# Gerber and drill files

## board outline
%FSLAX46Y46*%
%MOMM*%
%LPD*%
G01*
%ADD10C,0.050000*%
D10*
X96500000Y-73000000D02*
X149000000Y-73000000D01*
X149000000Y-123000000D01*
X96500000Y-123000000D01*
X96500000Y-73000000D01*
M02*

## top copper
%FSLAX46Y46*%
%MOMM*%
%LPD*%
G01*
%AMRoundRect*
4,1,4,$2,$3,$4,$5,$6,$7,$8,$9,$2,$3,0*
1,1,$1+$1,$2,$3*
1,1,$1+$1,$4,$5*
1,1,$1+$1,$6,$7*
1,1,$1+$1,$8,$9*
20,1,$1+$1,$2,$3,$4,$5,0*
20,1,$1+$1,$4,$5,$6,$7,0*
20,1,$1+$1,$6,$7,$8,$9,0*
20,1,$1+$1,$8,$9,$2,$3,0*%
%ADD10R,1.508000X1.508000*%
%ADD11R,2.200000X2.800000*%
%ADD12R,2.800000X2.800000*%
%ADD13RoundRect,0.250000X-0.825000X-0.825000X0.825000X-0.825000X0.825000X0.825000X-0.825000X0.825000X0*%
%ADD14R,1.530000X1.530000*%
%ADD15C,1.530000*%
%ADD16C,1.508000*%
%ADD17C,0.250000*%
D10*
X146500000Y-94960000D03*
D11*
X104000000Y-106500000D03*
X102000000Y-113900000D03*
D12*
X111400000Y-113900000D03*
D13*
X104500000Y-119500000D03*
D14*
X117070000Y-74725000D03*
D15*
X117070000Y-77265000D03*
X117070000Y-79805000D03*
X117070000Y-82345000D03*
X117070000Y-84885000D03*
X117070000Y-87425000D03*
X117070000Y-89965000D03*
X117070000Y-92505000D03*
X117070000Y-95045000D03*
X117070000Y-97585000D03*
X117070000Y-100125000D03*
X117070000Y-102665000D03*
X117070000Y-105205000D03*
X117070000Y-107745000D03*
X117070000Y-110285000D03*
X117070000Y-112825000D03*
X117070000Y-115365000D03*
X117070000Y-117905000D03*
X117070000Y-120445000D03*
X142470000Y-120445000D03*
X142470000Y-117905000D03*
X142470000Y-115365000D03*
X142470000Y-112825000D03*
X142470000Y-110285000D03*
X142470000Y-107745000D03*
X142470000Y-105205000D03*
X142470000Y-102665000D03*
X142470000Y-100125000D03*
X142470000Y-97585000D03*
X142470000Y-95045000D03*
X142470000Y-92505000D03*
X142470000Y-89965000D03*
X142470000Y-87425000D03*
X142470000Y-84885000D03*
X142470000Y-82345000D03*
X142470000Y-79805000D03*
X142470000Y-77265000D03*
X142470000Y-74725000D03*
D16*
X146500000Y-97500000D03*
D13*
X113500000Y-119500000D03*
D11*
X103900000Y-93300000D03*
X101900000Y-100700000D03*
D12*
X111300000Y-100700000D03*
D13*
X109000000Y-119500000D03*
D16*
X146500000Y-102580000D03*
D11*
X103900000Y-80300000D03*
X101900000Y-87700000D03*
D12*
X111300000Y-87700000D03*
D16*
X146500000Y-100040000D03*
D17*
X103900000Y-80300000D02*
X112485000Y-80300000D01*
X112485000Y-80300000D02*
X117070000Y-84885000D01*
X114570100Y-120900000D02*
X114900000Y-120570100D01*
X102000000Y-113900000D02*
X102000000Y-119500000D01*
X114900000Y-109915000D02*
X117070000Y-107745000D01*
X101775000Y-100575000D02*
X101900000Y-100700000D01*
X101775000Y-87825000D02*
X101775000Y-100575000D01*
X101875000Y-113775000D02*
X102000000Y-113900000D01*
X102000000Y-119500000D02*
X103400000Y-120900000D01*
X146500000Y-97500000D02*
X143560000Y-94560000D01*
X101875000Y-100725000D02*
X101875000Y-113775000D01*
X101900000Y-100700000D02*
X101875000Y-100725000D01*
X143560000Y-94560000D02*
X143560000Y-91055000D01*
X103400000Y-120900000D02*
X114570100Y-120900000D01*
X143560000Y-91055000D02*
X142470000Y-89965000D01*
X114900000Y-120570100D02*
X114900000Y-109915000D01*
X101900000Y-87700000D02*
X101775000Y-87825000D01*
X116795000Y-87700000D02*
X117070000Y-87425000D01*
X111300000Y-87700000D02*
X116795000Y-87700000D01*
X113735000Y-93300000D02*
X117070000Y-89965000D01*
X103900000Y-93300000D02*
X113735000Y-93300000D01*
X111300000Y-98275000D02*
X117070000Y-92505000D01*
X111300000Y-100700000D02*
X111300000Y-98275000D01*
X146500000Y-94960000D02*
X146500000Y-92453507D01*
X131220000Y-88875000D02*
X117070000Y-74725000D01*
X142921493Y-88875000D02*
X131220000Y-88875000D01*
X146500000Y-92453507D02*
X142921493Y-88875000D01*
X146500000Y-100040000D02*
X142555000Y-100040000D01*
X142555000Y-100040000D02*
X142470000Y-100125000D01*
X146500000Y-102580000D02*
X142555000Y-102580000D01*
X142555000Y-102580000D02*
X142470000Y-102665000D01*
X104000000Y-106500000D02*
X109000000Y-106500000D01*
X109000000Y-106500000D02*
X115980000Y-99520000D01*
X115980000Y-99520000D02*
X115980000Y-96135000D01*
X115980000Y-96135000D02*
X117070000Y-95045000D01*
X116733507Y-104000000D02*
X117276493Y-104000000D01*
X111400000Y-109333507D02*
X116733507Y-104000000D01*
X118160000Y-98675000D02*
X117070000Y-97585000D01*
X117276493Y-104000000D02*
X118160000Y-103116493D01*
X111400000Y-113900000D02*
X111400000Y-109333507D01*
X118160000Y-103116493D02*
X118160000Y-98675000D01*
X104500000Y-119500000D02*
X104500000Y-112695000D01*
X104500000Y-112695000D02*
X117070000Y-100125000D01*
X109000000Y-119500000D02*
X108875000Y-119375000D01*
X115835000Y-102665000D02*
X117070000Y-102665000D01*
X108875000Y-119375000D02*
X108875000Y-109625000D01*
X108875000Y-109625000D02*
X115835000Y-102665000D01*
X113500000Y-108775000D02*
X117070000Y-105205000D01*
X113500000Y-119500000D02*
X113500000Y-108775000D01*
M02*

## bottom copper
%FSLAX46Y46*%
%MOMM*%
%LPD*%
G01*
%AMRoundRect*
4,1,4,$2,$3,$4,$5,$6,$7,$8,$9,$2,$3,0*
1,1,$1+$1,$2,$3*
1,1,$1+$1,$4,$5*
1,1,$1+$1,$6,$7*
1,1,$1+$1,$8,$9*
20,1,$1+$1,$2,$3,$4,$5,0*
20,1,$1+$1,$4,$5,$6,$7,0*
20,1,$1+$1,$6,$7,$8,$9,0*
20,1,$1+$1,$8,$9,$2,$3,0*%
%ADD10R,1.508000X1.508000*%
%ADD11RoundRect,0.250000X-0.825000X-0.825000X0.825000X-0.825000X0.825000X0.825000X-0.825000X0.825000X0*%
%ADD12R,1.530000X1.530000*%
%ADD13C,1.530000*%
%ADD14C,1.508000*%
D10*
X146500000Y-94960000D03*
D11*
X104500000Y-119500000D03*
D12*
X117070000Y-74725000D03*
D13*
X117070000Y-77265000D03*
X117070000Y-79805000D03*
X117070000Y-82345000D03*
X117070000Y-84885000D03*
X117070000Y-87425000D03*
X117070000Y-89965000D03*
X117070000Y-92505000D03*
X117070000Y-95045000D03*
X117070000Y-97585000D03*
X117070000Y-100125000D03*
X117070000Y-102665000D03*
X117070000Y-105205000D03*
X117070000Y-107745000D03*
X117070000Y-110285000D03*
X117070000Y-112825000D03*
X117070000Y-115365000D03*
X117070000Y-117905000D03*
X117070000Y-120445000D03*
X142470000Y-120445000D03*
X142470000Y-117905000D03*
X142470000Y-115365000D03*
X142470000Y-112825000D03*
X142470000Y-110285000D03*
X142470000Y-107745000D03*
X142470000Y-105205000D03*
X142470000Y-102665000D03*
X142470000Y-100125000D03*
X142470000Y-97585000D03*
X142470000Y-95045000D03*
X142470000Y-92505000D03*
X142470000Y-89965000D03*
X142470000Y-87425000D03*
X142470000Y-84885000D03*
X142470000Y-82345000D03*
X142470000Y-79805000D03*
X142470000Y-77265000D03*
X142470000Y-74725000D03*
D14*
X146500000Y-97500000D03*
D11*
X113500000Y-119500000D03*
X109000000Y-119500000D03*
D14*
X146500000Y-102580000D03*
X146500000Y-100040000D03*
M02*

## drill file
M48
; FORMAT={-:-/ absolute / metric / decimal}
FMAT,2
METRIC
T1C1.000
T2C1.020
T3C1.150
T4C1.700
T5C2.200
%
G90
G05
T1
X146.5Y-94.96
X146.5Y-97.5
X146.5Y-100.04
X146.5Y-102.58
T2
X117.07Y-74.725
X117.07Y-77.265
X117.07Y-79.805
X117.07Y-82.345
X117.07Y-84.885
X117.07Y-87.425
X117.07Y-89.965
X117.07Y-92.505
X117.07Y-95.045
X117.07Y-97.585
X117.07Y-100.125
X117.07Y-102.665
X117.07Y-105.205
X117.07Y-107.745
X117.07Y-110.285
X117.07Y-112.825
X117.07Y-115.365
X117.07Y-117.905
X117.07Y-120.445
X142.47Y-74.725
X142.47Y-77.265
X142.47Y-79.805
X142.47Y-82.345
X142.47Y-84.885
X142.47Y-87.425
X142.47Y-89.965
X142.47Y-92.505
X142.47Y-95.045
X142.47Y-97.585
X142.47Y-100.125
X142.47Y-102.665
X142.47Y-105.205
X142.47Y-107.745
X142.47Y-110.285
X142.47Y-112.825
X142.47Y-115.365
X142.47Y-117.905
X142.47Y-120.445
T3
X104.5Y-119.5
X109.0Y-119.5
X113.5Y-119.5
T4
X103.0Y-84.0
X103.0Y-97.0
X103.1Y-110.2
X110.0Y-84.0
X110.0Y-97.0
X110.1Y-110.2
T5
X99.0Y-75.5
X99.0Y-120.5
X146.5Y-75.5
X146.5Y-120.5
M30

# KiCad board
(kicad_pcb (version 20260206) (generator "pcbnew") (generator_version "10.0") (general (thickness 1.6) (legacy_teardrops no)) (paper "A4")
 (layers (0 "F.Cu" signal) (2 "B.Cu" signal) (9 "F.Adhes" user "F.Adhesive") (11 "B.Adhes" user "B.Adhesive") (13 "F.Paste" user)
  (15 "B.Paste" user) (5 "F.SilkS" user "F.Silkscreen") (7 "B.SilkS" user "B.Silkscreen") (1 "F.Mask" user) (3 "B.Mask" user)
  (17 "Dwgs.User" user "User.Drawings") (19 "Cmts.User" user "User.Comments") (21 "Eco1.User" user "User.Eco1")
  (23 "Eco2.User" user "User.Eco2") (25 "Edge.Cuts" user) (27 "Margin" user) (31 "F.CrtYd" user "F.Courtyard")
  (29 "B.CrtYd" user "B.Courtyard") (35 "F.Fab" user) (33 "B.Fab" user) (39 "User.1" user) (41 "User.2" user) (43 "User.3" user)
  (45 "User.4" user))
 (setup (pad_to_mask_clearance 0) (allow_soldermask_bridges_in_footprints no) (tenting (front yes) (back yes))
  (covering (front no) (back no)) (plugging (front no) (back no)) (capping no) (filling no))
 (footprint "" (layer "F.Cu") (at 146.5 94.96 -90)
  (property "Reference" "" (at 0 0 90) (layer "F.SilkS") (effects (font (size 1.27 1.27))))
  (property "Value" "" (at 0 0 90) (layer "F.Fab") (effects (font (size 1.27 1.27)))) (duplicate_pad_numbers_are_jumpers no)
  (pad "1" thru_hole rect (at 0 0 270) (size 1.508 1.508) (drill 1) (layers "*.Cu" "*.Mask") (remove_unused_layers no) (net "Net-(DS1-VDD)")
   (solder_mask_margin 0.102)))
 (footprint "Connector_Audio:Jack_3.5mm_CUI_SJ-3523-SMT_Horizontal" (layer "F.Cu") (at 105.6 110.2 90)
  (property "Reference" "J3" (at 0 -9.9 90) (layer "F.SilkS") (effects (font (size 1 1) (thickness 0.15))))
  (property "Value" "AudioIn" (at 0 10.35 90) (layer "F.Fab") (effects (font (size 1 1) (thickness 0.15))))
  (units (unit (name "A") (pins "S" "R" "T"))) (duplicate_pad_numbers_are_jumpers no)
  (pad "" np_thru_hole circle (at 0 -2.5 90) (size 1.7 1.7) (drill 1.7) (layers "*.Cu" "*.Mask"))
  (pad "" np_thru_hole circle (at 0 4.5 90) (size 1.7 1.7) (drill 1.7) (layers "*.Cu" "*.Mask"))
  (pad "R" smd rect (at 3.7 -1.6 90) (size 2.8 2.2) (layers "F.Cu" "F.Mask" "F.Paste") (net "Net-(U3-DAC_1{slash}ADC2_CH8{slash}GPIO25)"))
  (pad "S" smd rect (at -3.7 -3.6 90) (size 2.8 2.2) (layers "F.Cu" "F.Mask" "F.Paste") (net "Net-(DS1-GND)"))
  (pad "T" smd rect (at -3.7 5.8 90) (size 2.8 2.8) (layers "F.Cu" "F.Mask" "F.Paste") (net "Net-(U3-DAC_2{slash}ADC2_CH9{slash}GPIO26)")))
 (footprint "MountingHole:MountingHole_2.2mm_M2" (layer "F.Cu") (at 99 120.5)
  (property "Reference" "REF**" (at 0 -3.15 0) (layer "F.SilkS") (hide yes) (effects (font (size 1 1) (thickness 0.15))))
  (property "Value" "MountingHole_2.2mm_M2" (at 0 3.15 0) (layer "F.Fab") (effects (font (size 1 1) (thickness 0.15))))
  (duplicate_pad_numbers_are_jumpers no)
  (pad "" np_thru_hole circle (at 0 0) (size 2.2 2.2) (drill 2.2) (layers "*.Cu" "*.Mask")))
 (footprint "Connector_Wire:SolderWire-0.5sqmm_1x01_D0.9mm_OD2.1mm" (layer "F.Cu") (at 104.5 119.5)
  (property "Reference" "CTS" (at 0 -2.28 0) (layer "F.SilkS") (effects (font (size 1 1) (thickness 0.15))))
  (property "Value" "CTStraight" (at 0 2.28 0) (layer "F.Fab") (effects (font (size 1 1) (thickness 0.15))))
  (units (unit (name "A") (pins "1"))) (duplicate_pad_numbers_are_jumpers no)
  (pad "1" thru_hole roundrect (at 0 0) (size 2.15 2.15) (drill 1.15) (layers "*.Cu" "*.Mask") (remove_unused_layers no)
   (roundrect_rratio 0.116279) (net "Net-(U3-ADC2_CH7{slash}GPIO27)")))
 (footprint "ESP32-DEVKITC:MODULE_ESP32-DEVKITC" (layer "F.Cu") (at 129.77 97.575)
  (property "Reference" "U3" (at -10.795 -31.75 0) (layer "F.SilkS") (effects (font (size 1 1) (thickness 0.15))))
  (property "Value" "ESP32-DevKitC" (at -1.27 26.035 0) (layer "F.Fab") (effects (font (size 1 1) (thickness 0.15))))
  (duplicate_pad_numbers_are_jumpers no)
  (pad "1" thru_hole rect (at -12.7 -22.85) (size 1.53 1.53) (drill 1.02) (layers "*.Cu" "*.Mask") (remove_unused_layers no)
   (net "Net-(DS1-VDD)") (solder_mask_margin 0.102))
  (pad "2" thru_hole circle (at -12.7 -20.31) (size 1.53 1.53) (drill 1.02) (layers "*.Cu" "*.Mask") (remove_unused_layers no)
   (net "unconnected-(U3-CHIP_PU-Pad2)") (solder_mask_margin 0.102))
  (pad "3" thru_hole circle (at -12.7 -17.77) (size 1.53 1.53) (drill 1.02) (layers "*.Cu" "*.Mask") (remove_unused_layers no)
   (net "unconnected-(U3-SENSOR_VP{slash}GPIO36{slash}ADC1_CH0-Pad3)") (solder_mask_margin 0.102))
  (pad "4" thru_hole circle (at -12.7 -15.23) (size 1.53 1.53) (drill 1.02) (layers "*.Cu" "*.Mask") (remove_unused_layers no)
   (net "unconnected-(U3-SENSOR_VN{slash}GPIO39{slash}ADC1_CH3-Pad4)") (solder_mask_margin 0.102))
  (pad "5" thru_hole circle (at -12.7 -12.69) (size 1.53 1.53) (drill 1.02) (layers "*.Cu" "*.Mask") (remove_unused_layers no)
   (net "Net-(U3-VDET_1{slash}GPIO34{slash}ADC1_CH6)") (solder_mask_margin 0.102))
  (pad "6" thru_hole circle (at -12.7 -10.15) (size 1.53 1.53) (drill 1.02) (layers "*.Cu" "*.Mask") (remove_unused_layers no)
   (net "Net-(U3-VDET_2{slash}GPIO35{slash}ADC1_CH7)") (solder_mask_margin 0.102))
  (pad "7" thru_hole circle (at -12.7 -7.61) (size 1.53 1.53) (drill 1.02) (layers "*.Cu" "*.Mask") (remove_unused_layers no)
   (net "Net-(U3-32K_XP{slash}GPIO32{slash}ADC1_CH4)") (solder_mask_margin 0.102))
  (pad "8" thru_hole circle (at -12.7 -5.07) (size 1.53 1.53) (drill 1.02) (layers "*.Cu" "*.Mask") (remove_unused_layers no)
   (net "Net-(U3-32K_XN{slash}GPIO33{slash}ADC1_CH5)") (solder_mask_margin 0.102))
  (pad "9" thru_hole circle (at -12.7 -2.53) (size 1.53 1.53) (drill 1.02) (layers "*.Cu" "*.Mask") (remove_unused_layers no)
   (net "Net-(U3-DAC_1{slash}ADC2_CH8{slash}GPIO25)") (solder_mask_margin 0.102))
  (pad "10" thru_hole circle (at -12.7 0.01) (size 1.53 1.53) (drill 1.02) (layers "*.Cu" "*.Mask") (remove_unused_layers no)
   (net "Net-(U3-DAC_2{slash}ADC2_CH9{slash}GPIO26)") (solder_mask_margin 0.102))
  (pad "11" thru_hole circle (at -12.7 2.55) (size 1.53 1.53) (drill 1.02) (layers "*.Cu" "*.Mask") (remove_unused_layers no)
   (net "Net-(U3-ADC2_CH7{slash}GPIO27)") (solder_mask_margin 0.102))
  (pad "12" thru_hole circle (at -12.7 5.09) (size 1.53 1.53) (drill 1.02) (layers "*.Cu" "*.Mask") (remove_unused_layers no)
   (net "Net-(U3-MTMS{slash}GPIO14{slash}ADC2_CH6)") (solder_mask_margin 0.102))
  (pad "13" thru_hole circle (at -12.7 7.63) (size 1.53 1.53) (drill 1.02) (layers "*.Cu" "*.Mask") (remove_unused_layers no)
   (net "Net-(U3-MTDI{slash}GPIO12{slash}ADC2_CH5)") (solder_mask_margin 0.102))
  (pad "14" thru_hole circle (at -12.7 10.17) (size 1.53 1.53) (drill 1.02) (layers "*.Cu" "*.Mask") (remove_unused_layers no)
   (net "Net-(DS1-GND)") (solder_mask_margin 0.102))
  (pad "15" thru_hole circle (at -12.7 12.71) (size 1.53 1.53) (drill 1.02) (layers "*.Cu" "*.Mask") (remove_unused_layers no)
   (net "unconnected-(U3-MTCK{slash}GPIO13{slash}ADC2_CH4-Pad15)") (solder_mask_margin 0.102))
  (pad "16" thru_hole circle (at -12.7 15.25) (size 1.53 1.53) (drill 1.02) (layers "*.Cu" "*.Mask") (remove_unused_layers no)
   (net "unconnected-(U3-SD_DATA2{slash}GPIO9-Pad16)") (solder_mask_margin 0.102))
  (pad "17" thru_hole circle (at -12.7 17.79) (size 1.53 1.53) (drill 1.02) (layers "*.Cu" "*.Mask") (remove_unused_layers no)
   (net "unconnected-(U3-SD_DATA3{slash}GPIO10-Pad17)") (solder_mask_margin 0.102))
  (pad "18" thru_hole circle (at -12.7 20.33) (size 1.53 1.53) (drill 1.02) (layers "*.Cu" "*.Mask") (remove_unused_layers no)
   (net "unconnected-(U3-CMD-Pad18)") (solder_mask_margin 0.102))
  (pad "19" thru_hole circle (at -12.7 22.87) (size 1.53 1.53) (drill 1.02) (layers "*.Cu" "*.Mask") (remove_unused_layers no)
   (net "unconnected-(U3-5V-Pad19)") (solder_mask_margin 0.102))
  (pad "20" thru_hole circle (at 12.7 22.87) (size 1.53 1.53) (drill 1.02) (layers "*.Cu" "*.Mask") (remove_unused_layers no)
   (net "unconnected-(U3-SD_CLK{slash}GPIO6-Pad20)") (solder_mask_margin 0.102))
  (pad "21" thru_hole circle (at 12.7 20.33) (size 1.53 1.53) (drill 1.02) (layers "*.Cu" "*.Mask") (remove_unused_layers no)
   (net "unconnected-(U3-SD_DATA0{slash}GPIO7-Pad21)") (solder_mask_margin 0.102))
  (pad "22" thru_hole circle (at 12.7 17.79) (size 1.53 1.53) (drill 1.02) (layers "*.Cu" "*.Mask") (remove_unused_layers no)
   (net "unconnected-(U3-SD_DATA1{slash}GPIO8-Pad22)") (solder_mask_margin 0.102))
  (pad "23" thru_hole circle (at 12.7 15.25) (size 1.53 1.53) (drill 1.02) (layers "*.Cu" "*.Mask") (remove_unused_layers no)
   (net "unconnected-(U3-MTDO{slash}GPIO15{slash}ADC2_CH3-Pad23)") (solder_mask_margin 0.102))
  (pad "24" thru_hole circle (at 12.7 12.71) (size 1.53 1.53) (drill 1.02) (layers "*.Cu" "*.Mask") (remove_unused_layers no)
   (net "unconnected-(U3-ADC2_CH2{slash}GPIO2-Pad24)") (solder_mask_margin 0.102))
  (pad "25" thru_hole circle (at 12.7 10.17) (size 1.53 1.53) (drill 1.02) (layers "*.Cu" "*.Mask") (remove_unused_layers no)
   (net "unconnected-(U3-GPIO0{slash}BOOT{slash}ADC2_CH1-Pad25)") (solder_mask_margin 0.102))
  (pad "26" thru_hole circle (at 12.7 7.63) (size 1.53 1.53) (drill 1.02) (layers "*.Cu" "*.Mask") (remove_unused_layers no)
   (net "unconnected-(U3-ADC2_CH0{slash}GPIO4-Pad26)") (solder_mask_margin 0.102))
  (pad "27" thru_hole circle (at 12.7 5.09) (size 1.53 1.53) (drill 1.02) (layers "*.Cu" "*.Mask") (remove_unused_layers no)
   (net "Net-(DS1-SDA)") (solder_mask_margin 0.102))
  (pad "28" thru_hole circle (at 12.7 2.55) (size 1.53 1.53) (drill 1.02) (layers "*.Cu" "*.Mask") (remove_unused_layers no)
   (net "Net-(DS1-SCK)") (solder_mask_margin 0.102))
  (pad "29" thru_hole circle (at 12.7 0.01) (size 1.53 1.53) (drill 1.02) (layers "*.Cu" "*.Mask") (remove_unused_layers no)
   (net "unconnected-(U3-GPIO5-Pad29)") (solder_mask_margin 0.102))
  (pad "30" thru_hole circle (at 12.7 -2.53) (size 1.53 1.53) (drill 1.02) (layers "*.Cu" "*.Mask") (remove_unused_layers no)
   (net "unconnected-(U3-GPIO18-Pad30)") (solder_mask_margin 0.102))
  (pad "31" thru_hole circle (at 12.7 -5.07) (size 1.53 1.53) (drill 1.02) (layers "*.Cu" "*.Mask") (remove_unused_layers no)
   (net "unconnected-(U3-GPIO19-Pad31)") (solder_mask_margin 0.102))
  (pad "32" thru_hole circle (at 12.7 -7.61) (size 1.53 1.53) (drill 1.02) (layers "*.Cu" "*.Mask") (remove_unused_layers no)
   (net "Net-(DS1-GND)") (solder_mask_margin 0.102))
  (pad "33" thru_hole circle (at 12.7 -10.15) (size 1.53 1.53) (drill 1.02) (layers "*.Cu" "*.Mask") (remove_unused_layers no)
   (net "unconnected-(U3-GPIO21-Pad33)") (solder_mask_margin 0.102))
  (pad "34" thru_hole circle (at 12.7 -12.69) (size 1.53 1.53) (drill 1.02) (layers "*.Cu" "*.Mask") (remove_unused_layers no)
   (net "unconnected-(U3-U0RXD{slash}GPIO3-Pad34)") (solder_mask_margin 0.102))
  (pad "35" thru_hole circle (at 12.7 -15.23) (size 1.53 1.53) (drill 1.02) (layers "*.Cu" "*.Mask") (remove_unused_layers no)
   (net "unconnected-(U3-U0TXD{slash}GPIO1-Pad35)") (solder_mask_margin 0.102))
  (pad "36" thru_hole circle (at 12.7 -17.77) (size 1.53 1.53) (drill 1.02) (layers "*.Cu" "*.Mask") (remove_unused_layers no)
   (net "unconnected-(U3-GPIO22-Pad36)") (solder_mask_margin 0.102))
  (pad "37" thru_hole circle (at 12.7 -20.31) (size 1.53 1.53) (drill 1.02) (layers "*.Cu" "*.Mask") (remove_unused_layers no)
   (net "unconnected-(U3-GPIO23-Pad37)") (solder_mask_margin 0.102))
  (pad "38" thru_hole circle (at 12.7 -22.85) (size 1.53 1.53) (drill 1.02) (layers "*.Cu" "*.Mask") (remove_unused_layers no)
   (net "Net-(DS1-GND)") (solder_mask_margin 0.102)))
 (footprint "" (layer "F.Cu") (at 146.5 97.5 -90)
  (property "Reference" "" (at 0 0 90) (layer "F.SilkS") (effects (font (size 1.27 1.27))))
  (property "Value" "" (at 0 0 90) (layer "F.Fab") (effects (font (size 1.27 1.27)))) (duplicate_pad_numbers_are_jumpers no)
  (pad "2" thru_hole circle (at 0 0 270) (size 1.508 1.508) (drill 1) (layers "*.Cu" "*.Mask") (remove_unused_layers no)
   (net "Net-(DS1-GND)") (solder_mask_margin 0.102)))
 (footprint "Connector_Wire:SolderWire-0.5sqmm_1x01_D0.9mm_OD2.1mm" (layer "F.Cu") (at 113.5 119.5)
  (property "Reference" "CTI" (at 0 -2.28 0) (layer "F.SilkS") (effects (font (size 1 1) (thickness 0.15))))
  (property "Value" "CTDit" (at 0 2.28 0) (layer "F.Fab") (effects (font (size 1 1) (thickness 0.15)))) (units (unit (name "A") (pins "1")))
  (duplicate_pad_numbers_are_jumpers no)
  (pad "1" thru_hole roundrect (at 0 0) (size 2.15 2.15) (drill 1.15) (layers "*.Cu" "*.Mask") (remove_unused_layers no)
   (roundrect_rratio 0.116279) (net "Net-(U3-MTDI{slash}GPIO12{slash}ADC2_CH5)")))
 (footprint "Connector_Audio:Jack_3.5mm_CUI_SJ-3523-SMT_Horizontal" (layer "F.Cu") (at 105.5 97 90)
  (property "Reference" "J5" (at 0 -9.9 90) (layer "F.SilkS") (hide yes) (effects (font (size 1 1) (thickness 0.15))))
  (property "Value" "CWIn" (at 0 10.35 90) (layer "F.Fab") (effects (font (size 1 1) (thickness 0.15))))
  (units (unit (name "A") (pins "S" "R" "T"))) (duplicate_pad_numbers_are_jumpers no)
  (pad "" np_thru_hole circle (at 0 -2.5 90) (size 1.7 1.7) (drill 1.7) (layers "*.Cu" "*.Mask"))
  (pad "" np_thru_hole circle (at 0 4.5 90) (size 1.7 1.7) (drill 1.7) (layers "*.Cu" "*.Mask"))
  (pad "R" smd rect (at 3.7 -1.6 90) (size 2.8 2.2) (layers "F.Cu" "F.Mask" "F.Paste") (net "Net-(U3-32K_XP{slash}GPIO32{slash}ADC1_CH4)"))
  (pad "S" smd rect (at -3.7 -3.6 90) (size 2.8 2.2) (layers "F.Cu" "F.Mask" "F.Paste") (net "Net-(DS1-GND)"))
  (pad "T" smd rect (at -3.7 5.8 90) (size 2.8 2.8) (layers "F.Cu" "F.Mask" "F.Paste") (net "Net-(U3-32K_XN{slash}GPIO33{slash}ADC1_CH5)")))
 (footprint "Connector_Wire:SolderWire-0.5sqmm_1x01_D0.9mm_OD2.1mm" (layer "F.Cu") (at 109 119.5)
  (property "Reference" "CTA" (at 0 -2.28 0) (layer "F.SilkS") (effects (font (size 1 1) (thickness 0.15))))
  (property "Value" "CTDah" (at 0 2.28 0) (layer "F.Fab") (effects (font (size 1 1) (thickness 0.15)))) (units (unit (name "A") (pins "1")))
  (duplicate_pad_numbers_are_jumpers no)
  (pad "1" thru_hole roundrect (at 0 0) (size 2.15 2.15) (drill 1.15) (layers "*.Cu" "*.Mask") (remove_unused_layers no)
   (roundrect_rratio 0.116279) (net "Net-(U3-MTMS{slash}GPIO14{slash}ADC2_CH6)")))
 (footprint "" (layer "F.Cu") (at 146.5 102.58 -90)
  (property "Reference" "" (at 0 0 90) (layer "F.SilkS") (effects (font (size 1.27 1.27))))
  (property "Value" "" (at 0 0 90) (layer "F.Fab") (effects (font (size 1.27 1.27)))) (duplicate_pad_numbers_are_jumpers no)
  (pad "4" thru_hole circle (at 0 0 270) (size 1.508 1.508) (drill 1) (layers "*.Cu" "*.Mask") (remove_unused_layers no)
   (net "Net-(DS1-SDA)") (solder_mask_margin 0.102)))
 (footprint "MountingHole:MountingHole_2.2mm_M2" (layer "F.Cu") (at 99 75.5)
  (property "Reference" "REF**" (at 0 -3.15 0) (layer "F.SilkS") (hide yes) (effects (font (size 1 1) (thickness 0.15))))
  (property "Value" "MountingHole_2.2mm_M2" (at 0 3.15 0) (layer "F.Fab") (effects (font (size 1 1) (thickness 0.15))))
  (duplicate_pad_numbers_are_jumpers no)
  (pad "" np_thru_hole circle (at 0 0) (size 2.2 2.2) (drill 2.2) (layers "*.Cu" "*.Mask")))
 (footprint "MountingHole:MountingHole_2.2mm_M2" (layer "F.Cu") (at 146.5 75.5)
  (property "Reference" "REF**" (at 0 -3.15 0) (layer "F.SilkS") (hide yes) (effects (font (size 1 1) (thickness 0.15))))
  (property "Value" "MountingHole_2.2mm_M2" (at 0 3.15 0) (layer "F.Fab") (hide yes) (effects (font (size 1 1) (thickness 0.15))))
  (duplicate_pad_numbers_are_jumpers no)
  (pad "" np_thru_hole circle (at 0 0) (size 2.2 2.2) (drill 2.2) (layers "*.Cu" "*.Mask")))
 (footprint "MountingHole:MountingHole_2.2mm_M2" (layer "F.Cu") (at 146.5 120.5)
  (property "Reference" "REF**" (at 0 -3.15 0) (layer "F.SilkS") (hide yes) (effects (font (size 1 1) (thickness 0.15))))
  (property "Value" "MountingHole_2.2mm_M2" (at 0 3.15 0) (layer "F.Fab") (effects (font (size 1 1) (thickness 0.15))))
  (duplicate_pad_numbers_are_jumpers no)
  (pad "" np_thru_hole circle (at 0 0) (size 2.2 2.2) (drill 2.2) (layers "*.Cu" "*.Mask")))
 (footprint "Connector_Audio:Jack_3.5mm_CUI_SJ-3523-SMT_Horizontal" (layer "F.Cu") (at 105.5 84 90)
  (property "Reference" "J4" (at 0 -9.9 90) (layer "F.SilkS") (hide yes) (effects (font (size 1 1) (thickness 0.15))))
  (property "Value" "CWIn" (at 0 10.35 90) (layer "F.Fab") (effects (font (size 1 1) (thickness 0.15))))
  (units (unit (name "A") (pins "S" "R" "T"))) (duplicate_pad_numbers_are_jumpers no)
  (pad "" np_thru_hole circle (at 0 -2.5 90) (size 1.7 1.7) (drill 1.7) (layers "*.Cu" "*.Mask"))
  (pad "" np_thru_hole circle (at 0 4.5 90) (size 1.7 1.7) (drill 1.7) (layers "*.Cu" "*.Mask"))
  (pad "R" smd rect (at 3.7 -1.6 90) (size 2.8 2.2) (layers "F.Cu" "F.Mask" "F.Paste") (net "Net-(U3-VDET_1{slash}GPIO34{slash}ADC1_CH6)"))
  (pad "S" smd rect (at -3.7 -3.6 90) (size 2.8 2.2) (layers "F.Cu" "F.Mask" "F.Paste") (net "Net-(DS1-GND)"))
  (pad "T" smd rect (at -3.7 5.8 90) (size 2.8 2.8) (layers "F.Cu" "F.Mask" "F.Paste") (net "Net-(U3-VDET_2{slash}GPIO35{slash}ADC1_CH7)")))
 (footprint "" (layer "F.Cu") (at 146.5 100.04 -90)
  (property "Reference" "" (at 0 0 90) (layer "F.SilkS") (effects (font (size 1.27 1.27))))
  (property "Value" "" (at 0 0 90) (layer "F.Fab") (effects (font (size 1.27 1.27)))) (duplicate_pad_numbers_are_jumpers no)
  (pad "3" thru_hole circle (at 0 0 270) (size 1.508 1.508) (drill 1) (layers "*.Cu" "*.Mask") (remove_unused_layers no)
   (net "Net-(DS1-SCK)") (solder_mask_margin 0.102)))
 (gr_rect (start 96.5 73) (end 149 123) (stroke (width 0.05) (type default)) (fill no) (layer "Edge.Cuts"))
 (segment (start 103.9 80.3) (end 112.485 80.3) (width 0.25) (layer "F.Cu") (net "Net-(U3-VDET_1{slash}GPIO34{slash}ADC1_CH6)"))
 (segment (start 112.485 80.3) (end 117.07 84.885) (width 0.25) (layer "F.Cu") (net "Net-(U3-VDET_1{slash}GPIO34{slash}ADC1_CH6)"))
 (segment (start 114.5701 120.9) (end 114.9 120.5701) (width 0.25) (layer "F.Cu") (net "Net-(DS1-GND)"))
 (segment (start 102 113.9) (end 102 119.5) (width 0.25) (layer "F.Cu") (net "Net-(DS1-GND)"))
 (segment (start 114.9 109.915) (end 117.07 107.745) (width 0.25) (layer "F.Cu") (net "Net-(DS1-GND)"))
 (segment (start 101.775 100.575) (end 101.9 100.7) (width 0.25) (layer "F.Cu") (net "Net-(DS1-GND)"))
 (segment (start 101.775 87.825) (end 101.775 100.575) (width 0.25) (layer "F.Cu") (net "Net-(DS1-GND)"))
 (segment (start 101.875 113.775) (end 102 113.9) (width 0.25) (layer "F.Cu") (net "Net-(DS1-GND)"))
 (segment (start 102 119.5) (end 103.4 120.9) (width 0.25) (layer "F.Cu") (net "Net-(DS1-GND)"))
 (segment (start 146.5 97.5) (end 143.56 94.56) (width 0.25) (layer "F.Cu") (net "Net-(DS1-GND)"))
 (segment (start 101.875 100.725) (end 101.875 113.775) (width 0.25) (layer "F.Cu") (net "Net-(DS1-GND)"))
 (segment (start 101.9 100.7) (end 101.875 100.725) (width 0.25) (layer "F.Cu") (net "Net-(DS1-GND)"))
 (segment (start 143.56 94.56) (end 143.56 91.055) (width 0.25) (layer "F.Cu") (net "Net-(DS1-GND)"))
 (segment (start 103.4 120.9) (end 114.5701 120.9) (width 0.25) (layer "F.Cu") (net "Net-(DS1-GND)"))
 (segment (start 143.56 91.055) (end 142.47 89.965) (width 0.25) (layer "F.Cu") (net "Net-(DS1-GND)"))
 (segment (start 114.9 120.5701) (end 114.9 109.915) (width 0.25) (layer "F.Cu") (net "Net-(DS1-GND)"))
 (segment (start 101.9 87.7) (end 101.775 87.825) (width 0.25) (layer "F.Cu") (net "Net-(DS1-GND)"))
 (segment (start 116.795 87.7) (end 117.07 87.425) (width 0.25) (layer "F.Cu") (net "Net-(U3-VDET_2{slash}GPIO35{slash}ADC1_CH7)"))
 (segment (start 111.3 87.7) (end 116.795 87.7) (width 0.25) (layer "F.Cu") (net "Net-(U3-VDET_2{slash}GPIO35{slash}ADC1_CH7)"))
 (segment (start 113.735 93.3) (end 117.07 89.965) (width 0.25) (layer "F.Cu") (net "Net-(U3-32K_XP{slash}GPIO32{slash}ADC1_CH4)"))
 (segment (start 103.9 93.3) (end 113.735 93.3) (width 0.25) (layer "F.Cu") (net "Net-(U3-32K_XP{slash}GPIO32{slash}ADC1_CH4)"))
 (segment (start 111.3 98.275) (end 117.07 92.505) (width 0.25) (layer "F.Cu") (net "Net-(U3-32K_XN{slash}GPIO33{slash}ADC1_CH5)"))
 (segment (start 111.3 100.7) (end 111.3 98.275) (width 0.25) (layer "F.Cu") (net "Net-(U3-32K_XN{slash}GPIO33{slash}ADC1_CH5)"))
 (segment (start 146.5 94.96) (end 146.5 92.453507) (width 0.25) (layer "F.Cu") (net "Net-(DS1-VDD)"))
 (segment (start 131.22 88.875) (end 117.07 74.725) (width 0.25) (layer "F.Cu") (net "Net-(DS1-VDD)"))
 (segment (start 142.921493 88.875) (end 131.22 88.875) (width 0.25) (layer "F.Cu") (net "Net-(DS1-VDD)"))
 (segment (start 146.5 92.453507) (end 142.921493 88.875) (width 0.25) (layer "F.Cu") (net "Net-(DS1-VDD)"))
 (segment (start 146.5 100.04) (end 142.555 100.04) (width 0.25) (layer "F.Cu") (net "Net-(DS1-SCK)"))
 (segment (start 142.555 100.04) (end 142.47 100.125) (width 0.25) (layer "F.Cu") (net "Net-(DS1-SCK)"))
 (segment (start 146.5 102.58) (end 142.555 102.58) (width 0.25) (layer "F.Cu") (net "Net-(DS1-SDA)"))
 (segment (start 142.555 102.58) (end 142.47 102.665) (width 0.25) (layer "F.Cu") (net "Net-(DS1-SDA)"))
 (segment (start 104 106.5) (end 109 106.5) (width 0.25) (layer "F.Cu") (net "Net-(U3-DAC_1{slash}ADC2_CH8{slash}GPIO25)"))
 (segment (start 109 106.5) (end 115.98 99.52) (width 0.25) (layer "F.Cu") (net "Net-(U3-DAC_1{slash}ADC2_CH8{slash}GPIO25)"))
 (segment (start 115.98 99.52) (end 115.98 96.135) (width 0.25) (layer "F.Cu") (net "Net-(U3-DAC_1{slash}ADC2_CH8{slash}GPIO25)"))
 (segment (start 115.98 96.135) (end 117.07 95.045) (width 0.25) (layer "F.Cu") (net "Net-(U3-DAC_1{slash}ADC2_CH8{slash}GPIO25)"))
 (segment (start 116.733507 104) (end 117.276493 104) (width 0.25) (layer "F.Cu") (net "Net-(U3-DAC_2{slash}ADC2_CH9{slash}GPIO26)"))
 (segment (start 111.4 109.333507) (end 116.733507 104) (width 0.25) (layer "F.Cu") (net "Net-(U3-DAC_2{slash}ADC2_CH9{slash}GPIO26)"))
 (segment (start 118.16 98.675) (end 117.07 97.585) (width 0.25) (layer "F.Cu") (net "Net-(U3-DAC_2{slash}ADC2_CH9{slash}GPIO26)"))
 (segment (start 117.276493 104) (end 118.16 103.116493) (width 0.25) (layer "F.Cu") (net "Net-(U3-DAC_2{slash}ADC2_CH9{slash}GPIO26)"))
 (segment (start 111.4 113.9) (end 111.4 109.333507) (width 0.25) (layer "F.Cu") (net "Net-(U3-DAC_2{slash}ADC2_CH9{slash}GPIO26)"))
 (segment (start 118.16 103.116493) (end 118.16 98.675) (width 0.25) (layer "F.Cu") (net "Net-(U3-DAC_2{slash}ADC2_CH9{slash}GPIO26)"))
 (segment (start 104.5 119.5) (end 104.5 112.695) (width 0.25) (layer "F.Cu") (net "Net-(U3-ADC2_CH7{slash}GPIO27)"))
 (segment (start 104.5 112.695) (end 117.07 100.125) (width 0.25) (layer "F.Cu") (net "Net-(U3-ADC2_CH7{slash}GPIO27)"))
 (segment (start 109 119.5) (end 108.875 119.375) (width 0.25) (layer "F.Cu") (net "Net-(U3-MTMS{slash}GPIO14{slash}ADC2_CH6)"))
 (segment (start 115.835 102.665) (end 117.07 102.665) (width 0.25) (layer "F.Cu") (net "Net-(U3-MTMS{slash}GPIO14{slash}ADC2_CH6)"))
 (segment (start 108.875 119.375) (end 108.875 109.625) (width 0.25) (layer "F.Cu") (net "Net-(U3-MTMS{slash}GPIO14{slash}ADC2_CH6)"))
 (segment (start 108.875 109.625) (end 115.835 102.665) (width 0.25) (layer "F.Cu") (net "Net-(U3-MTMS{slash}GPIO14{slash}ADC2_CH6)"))
 (segment (start 113.5 108.775) (end 117.07 105.205) (width 0.25) (layer "F.Cu") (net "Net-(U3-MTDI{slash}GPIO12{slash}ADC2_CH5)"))
 (segment (start 113.5 119.5) (end 113.5 108.775) (width 0.25) (layer "F.Cu") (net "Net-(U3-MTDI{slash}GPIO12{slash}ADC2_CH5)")))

